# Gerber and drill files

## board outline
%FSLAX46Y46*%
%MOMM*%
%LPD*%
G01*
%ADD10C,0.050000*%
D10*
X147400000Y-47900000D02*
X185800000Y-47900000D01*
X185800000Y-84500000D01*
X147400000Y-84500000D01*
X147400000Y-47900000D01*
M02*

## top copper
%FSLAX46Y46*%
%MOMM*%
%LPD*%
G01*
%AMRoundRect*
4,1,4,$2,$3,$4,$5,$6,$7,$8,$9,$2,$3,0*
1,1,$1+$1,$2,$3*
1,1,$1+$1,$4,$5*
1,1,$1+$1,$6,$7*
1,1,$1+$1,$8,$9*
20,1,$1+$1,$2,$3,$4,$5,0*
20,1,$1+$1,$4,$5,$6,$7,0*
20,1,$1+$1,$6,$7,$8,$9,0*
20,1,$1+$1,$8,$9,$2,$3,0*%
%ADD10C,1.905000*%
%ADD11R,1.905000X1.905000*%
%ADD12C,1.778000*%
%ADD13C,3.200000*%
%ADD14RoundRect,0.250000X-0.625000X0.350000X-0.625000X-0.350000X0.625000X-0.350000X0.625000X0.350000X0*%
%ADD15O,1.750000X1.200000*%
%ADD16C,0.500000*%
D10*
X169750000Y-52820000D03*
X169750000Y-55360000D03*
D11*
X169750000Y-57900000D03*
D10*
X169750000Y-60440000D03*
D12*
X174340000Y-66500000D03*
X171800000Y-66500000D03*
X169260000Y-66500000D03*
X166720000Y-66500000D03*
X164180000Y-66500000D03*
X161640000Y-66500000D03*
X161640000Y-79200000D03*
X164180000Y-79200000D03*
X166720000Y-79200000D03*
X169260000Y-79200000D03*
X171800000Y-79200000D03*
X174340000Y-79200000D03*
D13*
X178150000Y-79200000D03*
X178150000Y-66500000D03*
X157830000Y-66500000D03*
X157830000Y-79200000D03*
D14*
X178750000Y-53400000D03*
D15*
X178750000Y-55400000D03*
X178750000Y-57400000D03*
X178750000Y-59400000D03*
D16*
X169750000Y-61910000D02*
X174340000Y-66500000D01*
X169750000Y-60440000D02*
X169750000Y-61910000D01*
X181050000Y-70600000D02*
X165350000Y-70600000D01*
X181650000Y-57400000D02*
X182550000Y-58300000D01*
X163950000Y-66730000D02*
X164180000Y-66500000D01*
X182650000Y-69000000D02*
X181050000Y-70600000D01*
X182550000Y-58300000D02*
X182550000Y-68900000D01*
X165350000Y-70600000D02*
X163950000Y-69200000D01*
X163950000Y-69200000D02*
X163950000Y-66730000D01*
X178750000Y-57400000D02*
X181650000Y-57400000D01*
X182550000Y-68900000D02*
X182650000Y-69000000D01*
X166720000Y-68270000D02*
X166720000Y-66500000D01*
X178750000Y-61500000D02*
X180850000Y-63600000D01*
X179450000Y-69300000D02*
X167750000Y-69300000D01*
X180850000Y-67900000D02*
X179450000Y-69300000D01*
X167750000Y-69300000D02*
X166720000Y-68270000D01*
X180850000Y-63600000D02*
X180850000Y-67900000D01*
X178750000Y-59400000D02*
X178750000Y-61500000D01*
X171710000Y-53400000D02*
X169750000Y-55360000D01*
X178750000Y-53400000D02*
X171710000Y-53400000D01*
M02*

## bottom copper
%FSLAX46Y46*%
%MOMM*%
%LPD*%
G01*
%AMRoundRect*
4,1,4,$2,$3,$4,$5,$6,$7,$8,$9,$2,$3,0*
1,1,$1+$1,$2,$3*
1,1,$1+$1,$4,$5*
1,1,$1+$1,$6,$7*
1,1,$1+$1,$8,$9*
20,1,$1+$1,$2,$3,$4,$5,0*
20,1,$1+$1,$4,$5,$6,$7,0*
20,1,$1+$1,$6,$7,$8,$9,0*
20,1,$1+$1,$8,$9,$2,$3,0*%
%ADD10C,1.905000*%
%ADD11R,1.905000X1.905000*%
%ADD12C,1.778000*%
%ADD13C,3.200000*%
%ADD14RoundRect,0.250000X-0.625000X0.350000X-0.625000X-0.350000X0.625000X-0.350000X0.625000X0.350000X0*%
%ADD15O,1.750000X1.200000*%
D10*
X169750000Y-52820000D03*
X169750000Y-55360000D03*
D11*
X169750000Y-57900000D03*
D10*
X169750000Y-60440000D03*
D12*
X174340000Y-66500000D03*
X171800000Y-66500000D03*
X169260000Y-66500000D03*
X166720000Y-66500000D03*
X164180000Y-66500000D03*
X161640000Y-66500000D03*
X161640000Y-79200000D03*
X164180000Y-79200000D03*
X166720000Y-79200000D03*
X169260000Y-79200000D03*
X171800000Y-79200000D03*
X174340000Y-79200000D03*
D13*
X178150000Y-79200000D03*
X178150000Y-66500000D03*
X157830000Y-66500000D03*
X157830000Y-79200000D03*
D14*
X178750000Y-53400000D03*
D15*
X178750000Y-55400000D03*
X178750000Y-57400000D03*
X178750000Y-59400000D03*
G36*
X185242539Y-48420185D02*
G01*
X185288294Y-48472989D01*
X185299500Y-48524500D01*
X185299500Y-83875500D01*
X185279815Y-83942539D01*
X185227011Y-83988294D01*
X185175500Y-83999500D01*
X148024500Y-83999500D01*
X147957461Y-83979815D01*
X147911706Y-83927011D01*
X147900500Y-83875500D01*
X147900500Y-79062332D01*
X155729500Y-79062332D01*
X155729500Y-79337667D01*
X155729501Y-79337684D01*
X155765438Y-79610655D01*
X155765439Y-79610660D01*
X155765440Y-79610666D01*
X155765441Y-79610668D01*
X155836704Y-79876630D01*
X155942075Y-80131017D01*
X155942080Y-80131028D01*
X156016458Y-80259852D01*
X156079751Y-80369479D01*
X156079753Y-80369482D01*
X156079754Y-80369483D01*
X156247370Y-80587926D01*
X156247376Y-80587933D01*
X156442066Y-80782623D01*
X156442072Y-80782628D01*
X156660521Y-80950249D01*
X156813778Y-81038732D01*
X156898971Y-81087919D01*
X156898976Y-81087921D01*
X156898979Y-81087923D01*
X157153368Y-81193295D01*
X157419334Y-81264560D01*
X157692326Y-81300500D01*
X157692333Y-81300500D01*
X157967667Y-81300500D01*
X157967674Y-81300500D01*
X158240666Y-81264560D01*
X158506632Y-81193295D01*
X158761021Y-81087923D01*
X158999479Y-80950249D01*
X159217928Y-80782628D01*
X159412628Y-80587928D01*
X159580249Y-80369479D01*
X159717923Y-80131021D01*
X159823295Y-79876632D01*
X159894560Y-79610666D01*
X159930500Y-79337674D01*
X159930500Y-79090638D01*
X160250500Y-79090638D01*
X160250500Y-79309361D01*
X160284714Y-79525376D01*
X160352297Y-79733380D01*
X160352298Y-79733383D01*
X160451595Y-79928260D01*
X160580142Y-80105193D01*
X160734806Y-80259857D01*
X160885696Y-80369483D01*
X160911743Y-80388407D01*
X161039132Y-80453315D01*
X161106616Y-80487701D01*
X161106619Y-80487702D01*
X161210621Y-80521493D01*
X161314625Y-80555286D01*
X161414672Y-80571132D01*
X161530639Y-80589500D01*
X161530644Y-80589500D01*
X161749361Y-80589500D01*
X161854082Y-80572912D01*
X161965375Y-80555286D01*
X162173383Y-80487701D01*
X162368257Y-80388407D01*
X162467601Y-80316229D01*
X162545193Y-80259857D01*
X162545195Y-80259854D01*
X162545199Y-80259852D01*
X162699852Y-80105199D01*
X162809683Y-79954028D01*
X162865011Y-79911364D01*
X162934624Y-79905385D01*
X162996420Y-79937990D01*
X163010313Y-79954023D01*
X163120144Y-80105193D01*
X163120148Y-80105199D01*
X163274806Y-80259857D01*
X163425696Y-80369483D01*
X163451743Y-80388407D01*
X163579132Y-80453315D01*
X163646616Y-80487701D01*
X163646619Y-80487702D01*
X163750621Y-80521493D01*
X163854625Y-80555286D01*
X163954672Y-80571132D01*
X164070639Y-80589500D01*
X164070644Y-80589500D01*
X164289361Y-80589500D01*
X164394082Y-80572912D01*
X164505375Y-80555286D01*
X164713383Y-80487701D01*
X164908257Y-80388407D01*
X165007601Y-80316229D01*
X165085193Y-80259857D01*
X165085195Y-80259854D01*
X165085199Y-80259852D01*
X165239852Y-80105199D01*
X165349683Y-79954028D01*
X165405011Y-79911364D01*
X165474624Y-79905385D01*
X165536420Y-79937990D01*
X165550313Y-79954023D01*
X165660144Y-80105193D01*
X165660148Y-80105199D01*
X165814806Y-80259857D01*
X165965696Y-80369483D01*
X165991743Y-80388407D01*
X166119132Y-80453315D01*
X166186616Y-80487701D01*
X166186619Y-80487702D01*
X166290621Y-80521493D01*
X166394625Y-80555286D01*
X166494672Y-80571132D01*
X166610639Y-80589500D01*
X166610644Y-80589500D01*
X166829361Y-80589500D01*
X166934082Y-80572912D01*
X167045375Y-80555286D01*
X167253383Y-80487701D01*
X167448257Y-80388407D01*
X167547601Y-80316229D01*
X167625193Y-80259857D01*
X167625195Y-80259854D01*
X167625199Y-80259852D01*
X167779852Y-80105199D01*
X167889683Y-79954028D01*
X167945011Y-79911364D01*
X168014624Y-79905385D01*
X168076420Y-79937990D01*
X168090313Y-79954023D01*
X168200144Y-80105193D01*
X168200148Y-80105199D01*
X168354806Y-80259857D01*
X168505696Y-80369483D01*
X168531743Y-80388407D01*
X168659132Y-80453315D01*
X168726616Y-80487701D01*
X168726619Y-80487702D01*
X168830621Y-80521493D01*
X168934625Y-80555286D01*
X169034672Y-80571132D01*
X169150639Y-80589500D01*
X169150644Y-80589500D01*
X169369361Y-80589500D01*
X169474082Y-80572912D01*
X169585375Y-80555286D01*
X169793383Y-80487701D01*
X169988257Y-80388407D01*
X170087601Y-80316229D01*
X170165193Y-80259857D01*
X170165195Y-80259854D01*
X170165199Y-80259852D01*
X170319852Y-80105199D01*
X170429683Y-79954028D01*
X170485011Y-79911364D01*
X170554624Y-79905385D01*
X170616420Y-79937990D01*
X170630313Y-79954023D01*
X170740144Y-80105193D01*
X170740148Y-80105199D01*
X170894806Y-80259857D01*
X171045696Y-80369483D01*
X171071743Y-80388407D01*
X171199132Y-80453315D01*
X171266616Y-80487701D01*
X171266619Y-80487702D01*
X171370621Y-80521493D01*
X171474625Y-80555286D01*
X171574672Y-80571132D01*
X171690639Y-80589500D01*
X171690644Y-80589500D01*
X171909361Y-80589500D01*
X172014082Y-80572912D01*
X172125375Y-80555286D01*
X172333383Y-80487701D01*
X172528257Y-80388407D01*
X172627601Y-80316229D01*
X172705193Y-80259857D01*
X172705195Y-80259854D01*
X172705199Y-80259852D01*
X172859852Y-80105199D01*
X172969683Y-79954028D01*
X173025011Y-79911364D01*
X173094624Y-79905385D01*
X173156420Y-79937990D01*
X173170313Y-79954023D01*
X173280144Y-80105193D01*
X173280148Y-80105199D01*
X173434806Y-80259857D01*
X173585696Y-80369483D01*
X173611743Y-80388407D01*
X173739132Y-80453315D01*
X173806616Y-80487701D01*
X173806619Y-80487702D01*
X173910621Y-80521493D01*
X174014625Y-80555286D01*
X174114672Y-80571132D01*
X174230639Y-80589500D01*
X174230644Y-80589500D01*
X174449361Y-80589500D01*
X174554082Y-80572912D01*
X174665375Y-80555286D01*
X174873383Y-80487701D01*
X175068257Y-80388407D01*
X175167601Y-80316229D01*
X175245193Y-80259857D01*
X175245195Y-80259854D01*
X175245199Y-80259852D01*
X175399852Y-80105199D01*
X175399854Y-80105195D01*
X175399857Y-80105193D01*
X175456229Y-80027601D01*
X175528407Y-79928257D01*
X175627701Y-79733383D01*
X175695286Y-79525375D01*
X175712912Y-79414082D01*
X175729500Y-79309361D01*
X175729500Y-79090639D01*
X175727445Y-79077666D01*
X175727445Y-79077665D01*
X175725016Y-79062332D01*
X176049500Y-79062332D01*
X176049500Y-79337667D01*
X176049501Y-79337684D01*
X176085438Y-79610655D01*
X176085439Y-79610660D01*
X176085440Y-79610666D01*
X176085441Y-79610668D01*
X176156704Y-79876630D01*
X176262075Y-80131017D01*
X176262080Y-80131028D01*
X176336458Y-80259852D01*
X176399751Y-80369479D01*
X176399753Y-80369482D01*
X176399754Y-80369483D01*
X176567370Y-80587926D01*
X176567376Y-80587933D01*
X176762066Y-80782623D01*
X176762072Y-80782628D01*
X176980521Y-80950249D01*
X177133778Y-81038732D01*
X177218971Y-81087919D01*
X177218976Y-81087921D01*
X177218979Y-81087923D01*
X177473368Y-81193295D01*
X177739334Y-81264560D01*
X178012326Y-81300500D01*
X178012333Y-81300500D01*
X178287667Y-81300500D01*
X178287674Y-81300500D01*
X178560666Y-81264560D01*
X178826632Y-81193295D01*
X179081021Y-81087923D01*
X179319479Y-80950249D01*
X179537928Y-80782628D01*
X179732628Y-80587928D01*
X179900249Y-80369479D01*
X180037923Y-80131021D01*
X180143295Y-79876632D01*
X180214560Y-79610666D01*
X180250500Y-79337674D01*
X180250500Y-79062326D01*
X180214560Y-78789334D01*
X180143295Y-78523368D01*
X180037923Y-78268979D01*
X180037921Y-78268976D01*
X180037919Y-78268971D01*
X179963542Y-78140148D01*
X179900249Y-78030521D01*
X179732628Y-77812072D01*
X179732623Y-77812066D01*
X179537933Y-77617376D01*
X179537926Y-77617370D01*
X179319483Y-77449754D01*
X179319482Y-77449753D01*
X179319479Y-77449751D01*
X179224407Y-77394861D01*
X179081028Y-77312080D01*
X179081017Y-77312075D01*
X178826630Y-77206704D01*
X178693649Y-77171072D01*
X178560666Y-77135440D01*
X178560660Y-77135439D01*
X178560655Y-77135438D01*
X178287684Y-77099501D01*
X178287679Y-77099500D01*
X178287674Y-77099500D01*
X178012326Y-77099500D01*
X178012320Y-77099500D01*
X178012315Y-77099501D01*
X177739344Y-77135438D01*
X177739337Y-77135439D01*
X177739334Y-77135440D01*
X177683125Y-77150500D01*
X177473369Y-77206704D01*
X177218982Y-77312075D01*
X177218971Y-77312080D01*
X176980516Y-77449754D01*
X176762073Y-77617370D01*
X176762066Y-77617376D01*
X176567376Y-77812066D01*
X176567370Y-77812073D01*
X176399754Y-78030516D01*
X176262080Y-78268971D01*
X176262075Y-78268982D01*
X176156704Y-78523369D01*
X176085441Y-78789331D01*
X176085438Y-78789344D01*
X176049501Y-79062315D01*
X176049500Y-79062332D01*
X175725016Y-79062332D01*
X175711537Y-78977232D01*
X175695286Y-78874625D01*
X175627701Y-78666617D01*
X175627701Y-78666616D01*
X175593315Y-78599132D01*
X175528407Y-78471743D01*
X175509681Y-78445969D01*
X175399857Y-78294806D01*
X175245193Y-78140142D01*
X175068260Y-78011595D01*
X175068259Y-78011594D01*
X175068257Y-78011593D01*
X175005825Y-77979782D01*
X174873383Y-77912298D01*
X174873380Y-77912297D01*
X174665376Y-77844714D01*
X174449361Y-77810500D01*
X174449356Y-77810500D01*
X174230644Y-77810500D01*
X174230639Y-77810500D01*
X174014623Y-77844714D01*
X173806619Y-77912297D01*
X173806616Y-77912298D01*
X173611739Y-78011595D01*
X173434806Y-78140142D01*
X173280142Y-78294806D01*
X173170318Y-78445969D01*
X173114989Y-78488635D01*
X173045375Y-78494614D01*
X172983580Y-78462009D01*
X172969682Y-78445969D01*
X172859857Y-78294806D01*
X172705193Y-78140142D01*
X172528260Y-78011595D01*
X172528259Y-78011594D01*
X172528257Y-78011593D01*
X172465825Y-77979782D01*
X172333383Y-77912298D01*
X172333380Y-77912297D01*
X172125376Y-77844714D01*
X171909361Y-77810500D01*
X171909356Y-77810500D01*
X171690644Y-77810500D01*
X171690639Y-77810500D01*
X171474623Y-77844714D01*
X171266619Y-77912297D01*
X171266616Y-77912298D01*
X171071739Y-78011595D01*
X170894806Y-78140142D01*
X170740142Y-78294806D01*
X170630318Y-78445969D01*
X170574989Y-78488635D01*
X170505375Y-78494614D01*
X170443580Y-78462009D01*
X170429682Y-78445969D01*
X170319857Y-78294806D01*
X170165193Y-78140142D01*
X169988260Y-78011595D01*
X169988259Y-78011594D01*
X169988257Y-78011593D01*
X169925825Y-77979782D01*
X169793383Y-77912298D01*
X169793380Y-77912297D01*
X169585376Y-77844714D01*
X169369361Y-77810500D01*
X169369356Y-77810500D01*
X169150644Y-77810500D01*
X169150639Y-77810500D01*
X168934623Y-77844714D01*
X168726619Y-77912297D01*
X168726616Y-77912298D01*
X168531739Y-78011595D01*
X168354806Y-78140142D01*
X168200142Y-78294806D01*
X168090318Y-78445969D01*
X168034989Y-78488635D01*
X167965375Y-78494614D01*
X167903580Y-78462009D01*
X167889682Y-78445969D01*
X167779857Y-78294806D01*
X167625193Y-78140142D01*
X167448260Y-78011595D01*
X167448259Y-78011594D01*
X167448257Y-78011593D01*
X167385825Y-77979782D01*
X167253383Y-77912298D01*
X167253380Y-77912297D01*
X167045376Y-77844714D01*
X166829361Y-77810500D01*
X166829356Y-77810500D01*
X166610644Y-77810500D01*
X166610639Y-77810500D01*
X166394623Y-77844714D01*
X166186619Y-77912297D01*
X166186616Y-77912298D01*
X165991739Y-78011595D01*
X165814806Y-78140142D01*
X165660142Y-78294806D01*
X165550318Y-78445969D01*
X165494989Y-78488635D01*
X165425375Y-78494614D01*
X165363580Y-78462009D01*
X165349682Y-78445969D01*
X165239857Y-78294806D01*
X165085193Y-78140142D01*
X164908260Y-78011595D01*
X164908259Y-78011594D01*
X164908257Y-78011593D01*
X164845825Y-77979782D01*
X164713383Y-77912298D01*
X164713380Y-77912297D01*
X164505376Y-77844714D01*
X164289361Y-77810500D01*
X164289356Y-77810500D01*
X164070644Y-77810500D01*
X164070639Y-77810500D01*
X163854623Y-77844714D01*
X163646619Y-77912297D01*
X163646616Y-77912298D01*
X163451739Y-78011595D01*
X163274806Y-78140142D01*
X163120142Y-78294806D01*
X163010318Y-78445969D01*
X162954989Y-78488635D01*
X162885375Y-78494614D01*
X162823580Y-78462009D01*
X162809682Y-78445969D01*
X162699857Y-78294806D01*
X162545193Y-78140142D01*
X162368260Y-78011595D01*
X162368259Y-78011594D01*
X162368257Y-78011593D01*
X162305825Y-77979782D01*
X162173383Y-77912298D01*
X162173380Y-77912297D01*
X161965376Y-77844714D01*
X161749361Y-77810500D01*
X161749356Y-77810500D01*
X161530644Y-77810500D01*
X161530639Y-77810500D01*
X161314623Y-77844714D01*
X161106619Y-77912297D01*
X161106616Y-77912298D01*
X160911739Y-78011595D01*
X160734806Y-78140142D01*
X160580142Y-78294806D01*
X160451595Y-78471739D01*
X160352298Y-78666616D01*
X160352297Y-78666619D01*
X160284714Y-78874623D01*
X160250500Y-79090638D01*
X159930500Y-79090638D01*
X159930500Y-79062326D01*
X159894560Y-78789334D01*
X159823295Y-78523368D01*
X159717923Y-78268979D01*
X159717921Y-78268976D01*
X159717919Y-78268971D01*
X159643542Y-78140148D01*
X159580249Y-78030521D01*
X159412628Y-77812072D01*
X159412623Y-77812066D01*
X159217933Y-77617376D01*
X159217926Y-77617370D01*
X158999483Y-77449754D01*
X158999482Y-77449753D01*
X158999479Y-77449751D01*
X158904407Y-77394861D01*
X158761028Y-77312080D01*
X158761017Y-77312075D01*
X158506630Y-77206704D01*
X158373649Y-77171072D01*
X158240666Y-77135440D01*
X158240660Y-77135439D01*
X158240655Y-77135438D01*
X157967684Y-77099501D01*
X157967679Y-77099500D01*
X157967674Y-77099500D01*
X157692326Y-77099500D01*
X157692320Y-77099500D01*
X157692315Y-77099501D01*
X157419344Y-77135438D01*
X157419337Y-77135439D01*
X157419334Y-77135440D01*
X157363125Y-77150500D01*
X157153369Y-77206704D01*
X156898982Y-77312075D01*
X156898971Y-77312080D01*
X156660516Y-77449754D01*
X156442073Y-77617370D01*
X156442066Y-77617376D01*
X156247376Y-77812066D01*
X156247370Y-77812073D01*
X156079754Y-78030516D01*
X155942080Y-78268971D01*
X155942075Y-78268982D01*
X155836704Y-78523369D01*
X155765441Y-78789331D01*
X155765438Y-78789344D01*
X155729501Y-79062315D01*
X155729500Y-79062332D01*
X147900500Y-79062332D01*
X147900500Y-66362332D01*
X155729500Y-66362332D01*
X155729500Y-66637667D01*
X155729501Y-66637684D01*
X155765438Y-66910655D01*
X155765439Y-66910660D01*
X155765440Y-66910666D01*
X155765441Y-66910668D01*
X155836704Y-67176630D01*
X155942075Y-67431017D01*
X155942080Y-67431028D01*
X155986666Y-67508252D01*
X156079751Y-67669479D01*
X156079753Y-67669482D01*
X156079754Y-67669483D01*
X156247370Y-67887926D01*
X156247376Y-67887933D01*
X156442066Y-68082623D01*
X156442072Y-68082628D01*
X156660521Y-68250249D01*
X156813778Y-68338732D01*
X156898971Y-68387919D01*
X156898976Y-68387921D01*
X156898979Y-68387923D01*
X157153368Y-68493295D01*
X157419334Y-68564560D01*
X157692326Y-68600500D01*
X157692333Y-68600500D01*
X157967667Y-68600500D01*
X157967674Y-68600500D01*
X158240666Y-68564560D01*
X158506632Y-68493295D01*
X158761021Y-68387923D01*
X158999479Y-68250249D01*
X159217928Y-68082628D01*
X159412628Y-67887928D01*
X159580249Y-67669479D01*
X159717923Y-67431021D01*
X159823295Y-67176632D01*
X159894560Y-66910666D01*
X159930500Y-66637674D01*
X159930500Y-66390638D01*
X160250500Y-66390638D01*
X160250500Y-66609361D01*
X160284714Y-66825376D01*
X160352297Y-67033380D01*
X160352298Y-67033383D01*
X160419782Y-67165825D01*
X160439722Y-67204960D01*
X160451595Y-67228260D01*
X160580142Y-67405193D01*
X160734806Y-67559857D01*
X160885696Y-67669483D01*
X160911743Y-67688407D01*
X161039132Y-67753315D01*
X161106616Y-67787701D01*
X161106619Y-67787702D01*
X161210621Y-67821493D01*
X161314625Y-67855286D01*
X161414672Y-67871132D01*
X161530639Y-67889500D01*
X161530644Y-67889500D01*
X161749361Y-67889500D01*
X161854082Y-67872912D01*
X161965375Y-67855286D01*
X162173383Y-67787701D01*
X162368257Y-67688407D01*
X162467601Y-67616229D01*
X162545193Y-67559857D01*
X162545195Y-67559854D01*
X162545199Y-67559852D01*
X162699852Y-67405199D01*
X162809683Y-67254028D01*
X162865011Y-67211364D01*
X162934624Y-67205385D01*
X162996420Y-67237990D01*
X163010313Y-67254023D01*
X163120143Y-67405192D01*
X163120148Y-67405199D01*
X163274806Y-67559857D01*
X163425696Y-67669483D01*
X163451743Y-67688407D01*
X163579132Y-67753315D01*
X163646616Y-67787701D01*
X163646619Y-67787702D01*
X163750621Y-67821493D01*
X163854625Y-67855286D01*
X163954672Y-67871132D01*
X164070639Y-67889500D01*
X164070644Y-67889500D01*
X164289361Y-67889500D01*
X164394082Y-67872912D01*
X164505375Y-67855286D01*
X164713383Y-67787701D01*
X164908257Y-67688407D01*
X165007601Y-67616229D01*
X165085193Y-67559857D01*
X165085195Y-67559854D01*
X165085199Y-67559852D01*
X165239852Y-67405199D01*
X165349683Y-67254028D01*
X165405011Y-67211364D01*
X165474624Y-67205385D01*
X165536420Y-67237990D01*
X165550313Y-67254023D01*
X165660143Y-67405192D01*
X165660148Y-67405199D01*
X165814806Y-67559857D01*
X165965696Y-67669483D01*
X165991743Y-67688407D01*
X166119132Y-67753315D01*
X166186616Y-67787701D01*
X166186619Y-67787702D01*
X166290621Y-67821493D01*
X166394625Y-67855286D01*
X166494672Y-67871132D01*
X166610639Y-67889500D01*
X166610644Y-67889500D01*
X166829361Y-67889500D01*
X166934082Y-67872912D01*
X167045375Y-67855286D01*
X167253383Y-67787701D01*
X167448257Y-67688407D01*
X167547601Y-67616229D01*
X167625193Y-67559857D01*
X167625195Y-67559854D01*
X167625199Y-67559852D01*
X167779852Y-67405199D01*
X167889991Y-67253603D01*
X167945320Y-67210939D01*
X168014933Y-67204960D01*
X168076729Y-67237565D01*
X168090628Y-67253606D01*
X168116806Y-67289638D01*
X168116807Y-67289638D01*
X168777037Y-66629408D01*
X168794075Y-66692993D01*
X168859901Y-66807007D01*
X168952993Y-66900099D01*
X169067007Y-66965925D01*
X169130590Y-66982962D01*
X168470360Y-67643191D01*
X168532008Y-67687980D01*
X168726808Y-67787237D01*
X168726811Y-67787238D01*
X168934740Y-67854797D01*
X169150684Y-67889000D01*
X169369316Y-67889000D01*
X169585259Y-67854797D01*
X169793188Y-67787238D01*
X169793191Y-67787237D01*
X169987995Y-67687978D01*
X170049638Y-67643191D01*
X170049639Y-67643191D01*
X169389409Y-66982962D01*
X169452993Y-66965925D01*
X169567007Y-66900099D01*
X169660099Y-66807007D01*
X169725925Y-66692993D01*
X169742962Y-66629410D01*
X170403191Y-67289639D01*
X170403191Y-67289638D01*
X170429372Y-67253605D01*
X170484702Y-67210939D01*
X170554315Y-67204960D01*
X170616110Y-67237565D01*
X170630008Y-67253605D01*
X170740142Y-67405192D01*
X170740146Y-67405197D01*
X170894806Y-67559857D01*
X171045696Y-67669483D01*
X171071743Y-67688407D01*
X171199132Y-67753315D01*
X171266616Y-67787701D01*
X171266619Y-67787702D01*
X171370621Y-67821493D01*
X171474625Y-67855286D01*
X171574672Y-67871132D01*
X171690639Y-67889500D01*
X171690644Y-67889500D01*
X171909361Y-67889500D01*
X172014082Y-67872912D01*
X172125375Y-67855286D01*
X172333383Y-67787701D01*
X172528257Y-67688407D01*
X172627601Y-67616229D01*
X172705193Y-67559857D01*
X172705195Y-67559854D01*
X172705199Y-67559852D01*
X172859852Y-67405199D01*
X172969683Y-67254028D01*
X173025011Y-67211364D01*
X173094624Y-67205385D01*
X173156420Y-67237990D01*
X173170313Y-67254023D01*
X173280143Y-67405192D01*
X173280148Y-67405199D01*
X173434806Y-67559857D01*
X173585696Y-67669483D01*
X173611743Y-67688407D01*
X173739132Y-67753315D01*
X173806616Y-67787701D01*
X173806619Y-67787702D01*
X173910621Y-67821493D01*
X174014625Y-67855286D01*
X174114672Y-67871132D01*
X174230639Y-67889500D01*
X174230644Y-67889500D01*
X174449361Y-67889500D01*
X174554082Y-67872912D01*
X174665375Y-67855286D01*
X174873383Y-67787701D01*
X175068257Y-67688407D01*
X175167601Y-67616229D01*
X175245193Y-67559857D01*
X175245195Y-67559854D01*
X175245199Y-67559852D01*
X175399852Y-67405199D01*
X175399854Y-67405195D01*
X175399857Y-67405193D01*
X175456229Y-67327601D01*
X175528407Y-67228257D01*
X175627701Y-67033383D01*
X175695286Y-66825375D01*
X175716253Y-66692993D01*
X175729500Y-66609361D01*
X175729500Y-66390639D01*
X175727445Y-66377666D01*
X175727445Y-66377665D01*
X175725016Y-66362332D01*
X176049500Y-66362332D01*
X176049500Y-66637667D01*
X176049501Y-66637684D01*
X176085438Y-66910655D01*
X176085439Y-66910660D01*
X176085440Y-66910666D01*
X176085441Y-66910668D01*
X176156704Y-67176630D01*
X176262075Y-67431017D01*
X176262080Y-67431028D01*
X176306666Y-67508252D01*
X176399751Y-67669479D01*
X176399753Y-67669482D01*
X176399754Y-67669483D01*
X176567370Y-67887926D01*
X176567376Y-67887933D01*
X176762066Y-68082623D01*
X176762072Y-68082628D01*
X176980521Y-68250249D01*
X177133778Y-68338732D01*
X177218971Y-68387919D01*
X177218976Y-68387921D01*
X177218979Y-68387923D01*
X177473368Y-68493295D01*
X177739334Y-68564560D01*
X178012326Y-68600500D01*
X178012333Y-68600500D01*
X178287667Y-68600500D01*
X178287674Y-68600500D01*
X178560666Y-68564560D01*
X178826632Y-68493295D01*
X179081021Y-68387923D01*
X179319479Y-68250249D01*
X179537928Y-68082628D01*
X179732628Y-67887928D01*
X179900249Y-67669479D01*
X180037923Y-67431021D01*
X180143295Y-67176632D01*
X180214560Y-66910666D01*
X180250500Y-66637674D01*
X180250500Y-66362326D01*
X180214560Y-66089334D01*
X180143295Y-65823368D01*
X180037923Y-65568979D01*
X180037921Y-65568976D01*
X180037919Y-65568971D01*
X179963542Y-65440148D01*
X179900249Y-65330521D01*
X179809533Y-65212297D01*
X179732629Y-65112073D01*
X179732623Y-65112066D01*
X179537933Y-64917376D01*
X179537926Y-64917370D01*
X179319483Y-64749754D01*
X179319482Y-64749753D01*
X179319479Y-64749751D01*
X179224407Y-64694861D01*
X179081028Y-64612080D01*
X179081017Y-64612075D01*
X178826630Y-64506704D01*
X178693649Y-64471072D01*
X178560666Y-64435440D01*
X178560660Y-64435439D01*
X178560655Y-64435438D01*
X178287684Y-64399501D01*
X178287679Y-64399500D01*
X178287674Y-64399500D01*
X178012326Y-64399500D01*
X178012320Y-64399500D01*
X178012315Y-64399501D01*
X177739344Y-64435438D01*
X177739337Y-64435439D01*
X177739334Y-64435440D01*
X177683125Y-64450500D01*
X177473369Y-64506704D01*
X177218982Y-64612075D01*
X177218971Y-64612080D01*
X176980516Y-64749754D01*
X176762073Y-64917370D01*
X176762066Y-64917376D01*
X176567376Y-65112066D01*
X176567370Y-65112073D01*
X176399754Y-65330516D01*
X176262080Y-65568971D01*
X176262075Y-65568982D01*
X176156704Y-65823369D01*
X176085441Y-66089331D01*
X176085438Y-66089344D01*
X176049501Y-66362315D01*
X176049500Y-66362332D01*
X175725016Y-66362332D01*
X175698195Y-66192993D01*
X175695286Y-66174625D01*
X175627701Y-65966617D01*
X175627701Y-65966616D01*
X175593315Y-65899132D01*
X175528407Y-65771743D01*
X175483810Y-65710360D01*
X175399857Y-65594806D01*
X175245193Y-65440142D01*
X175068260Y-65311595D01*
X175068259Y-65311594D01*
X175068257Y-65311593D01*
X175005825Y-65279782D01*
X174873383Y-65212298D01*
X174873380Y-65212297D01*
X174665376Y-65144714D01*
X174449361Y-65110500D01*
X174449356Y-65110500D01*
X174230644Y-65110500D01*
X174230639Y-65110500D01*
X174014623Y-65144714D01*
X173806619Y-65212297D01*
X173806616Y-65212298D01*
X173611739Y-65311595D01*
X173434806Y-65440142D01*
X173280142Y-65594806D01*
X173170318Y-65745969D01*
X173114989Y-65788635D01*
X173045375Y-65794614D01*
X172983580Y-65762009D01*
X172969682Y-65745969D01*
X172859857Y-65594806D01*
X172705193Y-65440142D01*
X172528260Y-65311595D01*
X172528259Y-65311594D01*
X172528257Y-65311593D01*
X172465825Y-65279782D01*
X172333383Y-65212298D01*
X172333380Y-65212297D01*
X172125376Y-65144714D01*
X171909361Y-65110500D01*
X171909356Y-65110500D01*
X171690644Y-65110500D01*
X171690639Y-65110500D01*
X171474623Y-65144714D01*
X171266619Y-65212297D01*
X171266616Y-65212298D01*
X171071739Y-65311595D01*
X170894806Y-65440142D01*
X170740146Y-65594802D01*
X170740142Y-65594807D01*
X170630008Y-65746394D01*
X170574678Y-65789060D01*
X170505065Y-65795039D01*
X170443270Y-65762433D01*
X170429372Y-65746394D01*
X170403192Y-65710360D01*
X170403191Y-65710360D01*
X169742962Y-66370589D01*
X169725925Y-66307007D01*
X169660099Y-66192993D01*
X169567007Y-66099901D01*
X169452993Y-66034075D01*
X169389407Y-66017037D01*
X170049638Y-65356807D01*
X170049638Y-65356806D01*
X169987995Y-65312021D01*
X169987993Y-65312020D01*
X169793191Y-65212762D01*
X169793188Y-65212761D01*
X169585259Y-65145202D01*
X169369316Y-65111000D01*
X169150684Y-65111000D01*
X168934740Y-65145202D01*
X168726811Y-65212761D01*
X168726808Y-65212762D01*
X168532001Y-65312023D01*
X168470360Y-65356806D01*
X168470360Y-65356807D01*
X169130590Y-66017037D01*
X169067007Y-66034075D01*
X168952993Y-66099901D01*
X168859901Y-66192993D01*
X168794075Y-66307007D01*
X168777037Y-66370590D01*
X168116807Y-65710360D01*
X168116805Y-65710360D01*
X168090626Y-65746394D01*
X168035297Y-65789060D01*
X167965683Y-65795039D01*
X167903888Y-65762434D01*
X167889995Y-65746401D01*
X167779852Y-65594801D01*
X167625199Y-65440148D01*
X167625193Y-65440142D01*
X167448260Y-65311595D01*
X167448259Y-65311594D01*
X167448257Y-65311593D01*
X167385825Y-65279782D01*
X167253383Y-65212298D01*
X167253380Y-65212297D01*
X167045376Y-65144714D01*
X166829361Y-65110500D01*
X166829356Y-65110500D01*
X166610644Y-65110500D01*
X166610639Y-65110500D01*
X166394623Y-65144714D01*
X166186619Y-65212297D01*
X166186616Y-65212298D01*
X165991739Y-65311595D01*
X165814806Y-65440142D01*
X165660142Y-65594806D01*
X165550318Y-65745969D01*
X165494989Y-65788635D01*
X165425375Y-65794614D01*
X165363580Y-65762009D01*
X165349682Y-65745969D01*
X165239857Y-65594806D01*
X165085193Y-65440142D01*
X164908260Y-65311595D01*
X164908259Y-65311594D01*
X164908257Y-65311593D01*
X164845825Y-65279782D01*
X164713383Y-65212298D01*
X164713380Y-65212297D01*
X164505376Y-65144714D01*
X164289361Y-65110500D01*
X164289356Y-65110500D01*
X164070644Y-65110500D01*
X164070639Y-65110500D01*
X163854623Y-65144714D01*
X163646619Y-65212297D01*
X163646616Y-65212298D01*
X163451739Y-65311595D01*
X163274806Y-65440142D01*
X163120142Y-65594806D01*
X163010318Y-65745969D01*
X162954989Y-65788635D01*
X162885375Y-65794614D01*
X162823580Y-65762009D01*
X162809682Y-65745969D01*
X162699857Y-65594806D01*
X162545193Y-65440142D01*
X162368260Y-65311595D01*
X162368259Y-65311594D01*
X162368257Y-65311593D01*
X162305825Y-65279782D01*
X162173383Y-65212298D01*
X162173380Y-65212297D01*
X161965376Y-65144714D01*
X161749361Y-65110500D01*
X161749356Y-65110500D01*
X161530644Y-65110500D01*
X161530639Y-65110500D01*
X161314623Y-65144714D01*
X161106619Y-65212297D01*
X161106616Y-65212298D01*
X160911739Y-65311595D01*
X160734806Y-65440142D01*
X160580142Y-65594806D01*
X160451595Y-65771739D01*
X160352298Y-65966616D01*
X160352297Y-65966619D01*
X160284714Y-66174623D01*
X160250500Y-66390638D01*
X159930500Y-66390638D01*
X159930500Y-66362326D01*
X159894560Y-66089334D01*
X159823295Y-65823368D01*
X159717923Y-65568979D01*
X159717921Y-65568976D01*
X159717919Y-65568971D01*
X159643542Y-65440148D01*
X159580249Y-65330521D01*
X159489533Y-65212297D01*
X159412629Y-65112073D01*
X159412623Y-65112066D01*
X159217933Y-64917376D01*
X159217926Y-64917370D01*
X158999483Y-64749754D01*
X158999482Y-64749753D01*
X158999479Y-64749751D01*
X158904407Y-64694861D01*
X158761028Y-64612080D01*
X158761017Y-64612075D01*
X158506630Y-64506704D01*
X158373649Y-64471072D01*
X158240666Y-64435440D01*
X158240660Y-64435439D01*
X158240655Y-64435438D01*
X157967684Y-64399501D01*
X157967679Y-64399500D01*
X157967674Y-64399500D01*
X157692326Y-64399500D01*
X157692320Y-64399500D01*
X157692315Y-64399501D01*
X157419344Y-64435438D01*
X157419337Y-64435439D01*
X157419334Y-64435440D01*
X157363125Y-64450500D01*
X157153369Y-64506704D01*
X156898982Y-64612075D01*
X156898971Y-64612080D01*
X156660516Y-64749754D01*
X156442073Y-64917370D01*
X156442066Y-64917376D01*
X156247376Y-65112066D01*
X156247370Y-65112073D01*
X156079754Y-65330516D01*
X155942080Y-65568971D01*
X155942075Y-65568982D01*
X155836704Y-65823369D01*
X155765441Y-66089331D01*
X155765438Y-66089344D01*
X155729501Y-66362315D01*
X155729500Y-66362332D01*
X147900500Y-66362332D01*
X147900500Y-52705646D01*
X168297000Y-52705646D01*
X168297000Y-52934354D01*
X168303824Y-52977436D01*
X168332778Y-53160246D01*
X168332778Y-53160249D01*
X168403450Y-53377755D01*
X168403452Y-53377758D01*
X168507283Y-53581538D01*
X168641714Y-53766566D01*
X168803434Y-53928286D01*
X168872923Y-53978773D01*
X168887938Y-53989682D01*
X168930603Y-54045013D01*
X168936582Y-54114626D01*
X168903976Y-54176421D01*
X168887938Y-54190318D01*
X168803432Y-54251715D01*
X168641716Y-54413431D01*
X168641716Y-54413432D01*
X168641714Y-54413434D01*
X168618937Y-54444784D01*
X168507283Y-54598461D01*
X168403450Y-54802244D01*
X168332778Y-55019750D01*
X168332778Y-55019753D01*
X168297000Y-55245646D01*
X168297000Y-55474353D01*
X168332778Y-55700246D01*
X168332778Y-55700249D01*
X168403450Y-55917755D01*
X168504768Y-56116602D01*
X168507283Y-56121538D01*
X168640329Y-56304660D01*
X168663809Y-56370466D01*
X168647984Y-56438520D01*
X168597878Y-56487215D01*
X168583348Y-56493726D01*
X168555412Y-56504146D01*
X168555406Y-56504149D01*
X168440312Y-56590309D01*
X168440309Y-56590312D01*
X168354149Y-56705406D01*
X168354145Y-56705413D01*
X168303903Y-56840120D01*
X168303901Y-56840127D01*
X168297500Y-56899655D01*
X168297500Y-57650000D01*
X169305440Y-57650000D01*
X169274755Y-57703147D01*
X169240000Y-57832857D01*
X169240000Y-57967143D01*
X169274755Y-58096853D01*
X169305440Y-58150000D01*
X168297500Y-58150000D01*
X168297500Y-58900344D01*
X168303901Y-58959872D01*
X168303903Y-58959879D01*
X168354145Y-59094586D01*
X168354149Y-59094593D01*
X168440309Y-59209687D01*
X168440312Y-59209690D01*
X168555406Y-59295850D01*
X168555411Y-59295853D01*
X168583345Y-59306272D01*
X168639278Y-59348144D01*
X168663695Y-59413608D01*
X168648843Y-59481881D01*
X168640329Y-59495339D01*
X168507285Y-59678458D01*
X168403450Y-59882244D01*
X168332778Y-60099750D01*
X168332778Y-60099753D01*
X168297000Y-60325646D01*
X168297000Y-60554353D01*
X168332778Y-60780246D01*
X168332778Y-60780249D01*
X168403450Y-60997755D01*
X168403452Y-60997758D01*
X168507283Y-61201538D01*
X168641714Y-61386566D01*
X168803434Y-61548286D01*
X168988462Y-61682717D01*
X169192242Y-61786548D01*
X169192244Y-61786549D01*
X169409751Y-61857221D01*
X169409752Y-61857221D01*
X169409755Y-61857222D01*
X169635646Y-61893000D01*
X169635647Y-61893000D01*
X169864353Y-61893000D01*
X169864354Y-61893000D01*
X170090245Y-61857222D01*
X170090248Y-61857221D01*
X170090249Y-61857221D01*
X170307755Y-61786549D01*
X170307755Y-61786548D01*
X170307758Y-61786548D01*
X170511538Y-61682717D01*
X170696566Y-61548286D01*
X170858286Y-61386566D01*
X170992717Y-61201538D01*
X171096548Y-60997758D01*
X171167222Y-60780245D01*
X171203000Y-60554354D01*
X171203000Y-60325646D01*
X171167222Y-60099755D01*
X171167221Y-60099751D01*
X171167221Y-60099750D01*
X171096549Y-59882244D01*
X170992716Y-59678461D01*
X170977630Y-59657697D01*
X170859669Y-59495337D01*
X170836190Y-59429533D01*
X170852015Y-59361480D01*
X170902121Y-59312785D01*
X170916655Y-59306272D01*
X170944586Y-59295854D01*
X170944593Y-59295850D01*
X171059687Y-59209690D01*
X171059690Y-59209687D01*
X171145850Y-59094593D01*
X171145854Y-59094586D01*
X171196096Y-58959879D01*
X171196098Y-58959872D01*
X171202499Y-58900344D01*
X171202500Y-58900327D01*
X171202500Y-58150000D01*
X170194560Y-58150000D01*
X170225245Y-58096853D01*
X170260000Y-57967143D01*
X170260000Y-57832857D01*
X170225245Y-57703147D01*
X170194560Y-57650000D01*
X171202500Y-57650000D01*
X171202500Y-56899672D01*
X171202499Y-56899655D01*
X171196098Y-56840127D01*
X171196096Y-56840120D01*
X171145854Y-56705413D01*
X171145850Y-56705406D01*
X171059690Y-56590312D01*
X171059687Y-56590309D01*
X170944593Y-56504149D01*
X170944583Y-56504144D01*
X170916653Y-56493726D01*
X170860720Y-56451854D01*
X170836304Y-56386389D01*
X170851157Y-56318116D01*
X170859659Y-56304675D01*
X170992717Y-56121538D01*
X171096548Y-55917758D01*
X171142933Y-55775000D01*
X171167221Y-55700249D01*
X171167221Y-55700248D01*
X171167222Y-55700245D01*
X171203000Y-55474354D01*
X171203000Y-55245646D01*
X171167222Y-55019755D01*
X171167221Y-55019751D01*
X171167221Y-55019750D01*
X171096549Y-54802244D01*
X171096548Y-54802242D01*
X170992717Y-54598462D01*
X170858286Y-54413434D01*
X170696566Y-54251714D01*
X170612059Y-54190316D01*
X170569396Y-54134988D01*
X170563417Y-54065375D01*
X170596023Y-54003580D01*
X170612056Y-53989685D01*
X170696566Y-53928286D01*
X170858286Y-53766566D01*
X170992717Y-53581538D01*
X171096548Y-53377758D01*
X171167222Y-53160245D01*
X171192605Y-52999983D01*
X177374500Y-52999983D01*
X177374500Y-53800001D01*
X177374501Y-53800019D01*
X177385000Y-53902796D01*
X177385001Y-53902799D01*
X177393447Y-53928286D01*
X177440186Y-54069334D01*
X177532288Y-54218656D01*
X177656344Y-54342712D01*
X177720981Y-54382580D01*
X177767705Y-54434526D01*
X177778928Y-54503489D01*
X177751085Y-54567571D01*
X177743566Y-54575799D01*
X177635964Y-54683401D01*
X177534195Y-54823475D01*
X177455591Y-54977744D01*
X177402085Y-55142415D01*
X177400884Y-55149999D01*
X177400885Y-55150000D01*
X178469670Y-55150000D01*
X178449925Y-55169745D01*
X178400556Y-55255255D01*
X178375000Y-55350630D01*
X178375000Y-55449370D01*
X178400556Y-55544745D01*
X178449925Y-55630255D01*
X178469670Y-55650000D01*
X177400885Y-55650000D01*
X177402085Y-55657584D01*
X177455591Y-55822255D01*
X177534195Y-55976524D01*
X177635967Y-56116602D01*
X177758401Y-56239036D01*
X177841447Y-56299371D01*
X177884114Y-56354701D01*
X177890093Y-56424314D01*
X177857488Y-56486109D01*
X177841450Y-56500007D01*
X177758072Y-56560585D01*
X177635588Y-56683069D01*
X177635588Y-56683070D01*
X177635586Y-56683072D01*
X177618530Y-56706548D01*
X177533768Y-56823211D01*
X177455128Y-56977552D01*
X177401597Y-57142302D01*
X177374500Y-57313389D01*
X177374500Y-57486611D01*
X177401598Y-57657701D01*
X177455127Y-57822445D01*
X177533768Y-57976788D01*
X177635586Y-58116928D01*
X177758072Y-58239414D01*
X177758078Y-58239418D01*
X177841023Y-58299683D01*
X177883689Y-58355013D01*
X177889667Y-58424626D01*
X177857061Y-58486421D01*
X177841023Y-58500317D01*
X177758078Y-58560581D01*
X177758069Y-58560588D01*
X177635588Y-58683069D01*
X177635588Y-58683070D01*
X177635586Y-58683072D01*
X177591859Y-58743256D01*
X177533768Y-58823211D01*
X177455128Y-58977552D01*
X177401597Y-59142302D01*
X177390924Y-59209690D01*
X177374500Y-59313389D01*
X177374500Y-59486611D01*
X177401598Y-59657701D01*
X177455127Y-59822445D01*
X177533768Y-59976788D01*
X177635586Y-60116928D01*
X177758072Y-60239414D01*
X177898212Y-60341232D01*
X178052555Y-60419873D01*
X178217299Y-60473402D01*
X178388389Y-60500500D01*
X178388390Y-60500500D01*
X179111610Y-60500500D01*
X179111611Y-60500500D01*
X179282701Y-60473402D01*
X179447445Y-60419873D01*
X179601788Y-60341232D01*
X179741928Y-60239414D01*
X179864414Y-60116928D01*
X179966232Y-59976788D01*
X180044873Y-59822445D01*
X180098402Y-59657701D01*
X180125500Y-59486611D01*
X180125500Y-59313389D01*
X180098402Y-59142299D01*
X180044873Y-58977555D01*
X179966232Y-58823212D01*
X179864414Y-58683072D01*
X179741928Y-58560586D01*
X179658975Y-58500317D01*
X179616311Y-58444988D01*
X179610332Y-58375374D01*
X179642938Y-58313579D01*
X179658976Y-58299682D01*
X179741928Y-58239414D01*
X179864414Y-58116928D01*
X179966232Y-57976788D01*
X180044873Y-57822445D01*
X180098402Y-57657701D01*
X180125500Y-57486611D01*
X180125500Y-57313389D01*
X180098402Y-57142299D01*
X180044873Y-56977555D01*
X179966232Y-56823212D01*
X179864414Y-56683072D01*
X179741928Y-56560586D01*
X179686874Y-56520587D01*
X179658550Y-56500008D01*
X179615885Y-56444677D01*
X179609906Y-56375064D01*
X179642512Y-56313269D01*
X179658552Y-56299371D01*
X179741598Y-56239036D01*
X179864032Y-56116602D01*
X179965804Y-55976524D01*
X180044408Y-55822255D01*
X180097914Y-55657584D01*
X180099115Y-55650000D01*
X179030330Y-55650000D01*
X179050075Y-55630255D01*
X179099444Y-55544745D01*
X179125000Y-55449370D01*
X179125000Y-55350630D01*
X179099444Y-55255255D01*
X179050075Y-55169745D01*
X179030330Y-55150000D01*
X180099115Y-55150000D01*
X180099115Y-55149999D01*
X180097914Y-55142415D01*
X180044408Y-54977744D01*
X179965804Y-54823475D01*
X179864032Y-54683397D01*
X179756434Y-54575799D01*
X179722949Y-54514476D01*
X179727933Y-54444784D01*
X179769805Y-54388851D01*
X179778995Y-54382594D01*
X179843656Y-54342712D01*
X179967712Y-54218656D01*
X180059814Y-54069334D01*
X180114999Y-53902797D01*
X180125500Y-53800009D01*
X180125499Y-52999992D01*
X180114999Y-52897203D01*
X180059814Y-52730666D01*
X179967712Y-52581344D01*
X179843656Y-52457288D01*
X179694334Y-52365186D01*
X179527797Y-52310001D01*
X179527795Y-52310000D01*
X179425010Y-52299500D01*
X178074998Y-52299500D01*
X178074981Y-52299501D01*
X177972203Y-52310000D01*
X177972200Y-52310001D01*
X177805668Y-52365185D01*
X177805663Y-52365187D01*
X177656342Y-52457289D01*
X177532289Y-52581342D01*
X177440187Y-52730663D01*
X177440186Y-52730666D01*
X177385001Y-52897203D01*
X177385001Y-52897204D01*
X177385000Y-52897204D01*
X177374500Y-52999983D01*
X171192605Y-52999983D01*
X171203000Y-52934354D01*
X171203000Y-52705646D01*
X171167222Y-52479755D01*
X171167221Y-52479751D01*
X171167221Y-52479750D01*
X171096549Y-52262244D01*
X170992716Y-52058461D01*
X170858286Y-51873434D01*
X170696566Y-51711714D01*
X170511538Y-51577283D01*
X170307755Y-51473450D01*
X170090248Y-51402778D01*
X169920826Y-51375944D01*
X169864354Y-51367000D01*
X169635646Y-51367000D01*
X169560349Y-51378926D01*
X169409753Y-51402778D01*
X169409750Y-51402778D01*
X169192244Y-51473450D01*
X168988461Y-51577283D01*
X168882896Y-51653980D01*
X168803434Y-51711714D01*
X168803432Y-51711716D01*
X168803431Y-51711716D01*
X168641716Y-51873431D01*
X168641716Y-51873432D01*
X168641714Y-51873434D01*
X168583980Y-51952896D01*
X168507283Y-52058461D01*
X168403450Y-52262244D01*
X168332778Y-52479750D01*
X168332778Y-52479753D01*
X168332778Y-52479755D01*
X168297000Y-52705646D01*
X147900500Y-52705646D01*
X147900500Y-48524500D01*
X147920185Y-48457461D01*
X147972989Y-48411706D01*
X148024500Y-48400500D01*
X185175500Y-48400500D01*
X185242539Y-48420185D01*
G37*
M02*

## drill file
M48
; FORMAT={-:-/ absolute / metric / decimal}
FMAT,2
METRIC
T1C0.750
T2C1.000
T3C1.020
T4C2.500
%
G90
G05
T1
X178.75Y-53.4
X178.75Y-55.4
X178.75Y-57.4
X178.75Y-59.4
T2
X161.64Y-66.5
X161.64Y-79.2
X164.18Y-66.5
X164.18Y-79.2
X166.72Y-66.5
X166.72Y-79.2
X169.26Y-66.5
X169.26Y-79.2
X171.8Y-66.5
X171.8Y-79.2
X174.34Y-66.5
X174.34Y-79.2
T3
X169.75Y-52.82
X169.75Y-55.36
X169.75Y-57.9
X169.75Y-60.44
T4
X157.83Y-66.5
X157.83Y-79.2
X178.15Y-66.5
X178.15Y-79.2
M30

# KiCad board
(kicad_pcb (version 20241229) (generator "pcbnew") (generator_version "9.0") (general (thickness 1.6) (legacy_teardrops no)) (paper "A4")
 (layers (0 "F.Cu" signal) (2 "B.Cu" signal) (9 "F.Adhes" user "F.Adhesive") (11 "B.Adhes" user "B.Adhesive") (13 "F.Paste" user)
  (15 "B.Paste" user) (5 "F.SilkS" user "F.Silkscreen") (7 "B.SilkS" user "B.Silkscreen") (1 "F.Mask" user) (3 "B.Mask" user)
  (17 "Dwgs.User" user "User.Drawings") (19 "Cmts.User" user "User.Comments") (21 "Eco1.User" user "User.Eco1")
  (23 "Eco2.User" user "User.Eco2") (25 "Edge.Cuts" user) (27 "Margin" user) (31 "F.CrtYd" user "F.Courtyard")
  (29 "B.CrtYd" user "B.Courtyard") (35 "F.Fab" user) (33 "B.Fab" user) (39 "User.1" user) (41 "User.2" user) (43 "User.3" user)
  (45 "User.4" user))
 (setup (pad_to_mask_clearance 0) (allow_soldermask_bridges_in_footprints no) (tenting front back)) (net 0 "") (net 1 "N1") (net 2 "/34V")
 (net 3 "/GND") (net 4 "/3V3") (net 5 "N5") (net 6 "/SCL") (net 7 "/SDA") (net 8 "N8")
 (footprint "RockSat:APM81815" (layer "F.Cu") (at 151.92 61.75 90)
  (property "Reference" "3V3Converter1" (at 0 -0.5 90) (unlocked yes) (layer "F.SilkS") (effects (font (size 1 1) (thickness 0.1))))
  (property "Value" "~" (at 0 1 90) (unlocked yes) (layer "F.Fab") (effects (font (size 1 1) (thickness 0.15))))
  (pad "1" thru_hole circle (at 8.93 17.83 90) (size 1.905 1.905) (drill 1.02) (layers "*.Cu" "*.Mask") (remove_unused_layers no)
   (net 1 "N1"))
  (pad "2" thru_hole circle (at 6.39 17.83 90) (size 1.905 1.905) (drill 1.02) (layers "*.Cu" "*.Mask") (remove_unused_layers no)
   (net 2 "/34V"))
  (pad "3" thru_hole rect (at 3.85 17.83 90) (size 1.905 1.905) (drill 1.02) (layers "*.Cu" "*.Mask") (remove_unused_layers no)
   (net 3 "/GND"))
  (pad "4" thru_hole circle (at 1.31 17.83 90) (size 1.905 1.905) (drill 1.02) (layers "*.Cu" "*.Mask") (remove_unused_layers no)
   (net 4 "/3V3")))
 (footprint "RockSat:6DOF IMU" (layer "F.Cu") (at 167.99 72.85 180)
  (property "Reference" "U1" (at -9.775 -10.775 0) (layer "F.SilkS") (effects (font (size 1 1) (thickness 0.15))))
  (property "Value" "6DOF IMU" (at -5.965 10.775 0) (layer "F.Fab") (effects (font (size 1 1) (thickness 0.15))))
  (pad "JP1_1" thru_hole circle (at -6.35 6.35 180) (size 1.778 1.778) (drill 1) (layers "*.Cu" "*.Mask") (remove_unused_layers no)
   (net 4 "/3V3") (solder_mask_margin 0.102))
  (pad "JP1_2" thru_hole circle (at -3.81 6.35 180) (size 1.778 1.778) (drill 1) (layers "*.Cu" "*.Mask") (remove_unused_layers no)
   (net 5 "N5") (solder_mask_margin 0.102))
  (pad "JP1_3" thru_hole circle (at -1.27 6.35 180) (size 1.778 1.778) (drill 1) (layers "*.Cu" "*.Mask") (remove_unused_layers no)
   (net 3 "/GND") (solder_mask_margin 0.102))
  (pad "JP1_4" thru_hole circle (at 1.27 6.35 180) (size 1.778 1.778) (drill 1) (layers "*.Cu" "*.Mask") (remove_unused_layers no)
   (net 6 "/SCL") (solder_mask_margin 0.102))
  (pad "JP1_5" thru_hole circle (at 3.81 6.35 180) (size 1.778 1.778) (drill 1) (layers "*.Cu" "*.Mask") (remove_unused_layers no)
   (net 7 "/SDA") (solder_mask_margin 0.102))
  (pad "JP1_6" thru_hole circle (at 6.35 6.35 180) (size 1.778 1.778) (drill 1) (layers "*.Cu" "*.Mask") (remove_unused_layers no)
   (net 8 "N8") (solder_mask_margin 0.102))
  (pad "JP3_1" thru_hole circle (at 6.35 -6.35 180) (size 1.778 1.778) (drill 1) (layers "*.Cu" "*.Mask") (remove_unused_layers no)
   (solder_mask_margin 0.102))
  (pad "JP3_2" thru_hole circle (at 3.81 -6.35 180) (size 1.778 1.778) (drill 1) (layers "*.Cu" "*.Mask") (remove_unused_layers no)
   (solder_mask_margin 0.102))
  (pad "JP3_3" thru_hole circle (at 1.27 -6.35 180) (size 1.778 1.778) (drill 1) (layers "*.Cu" "*.Mask") (remove_unused_layers no)
   (solder_mask_margin 0.102))
  (pad "JP3_4" thru_hole circle (at -1.27 -6.35 180) (size 1.778 1.778) (drill 1) (layers "*.Cu" "*.Mask") (remove_unused_layers no)
   (solder_mask_margin 0.102))
  (pad "JP3_5" thru_hole circle (at -3.81 -6.35 180) (size 1.778 1.778) (drill 1) (layers "*.Cu" "*.Mask") (remove_unused_layers no)
   (solder_mask_margin 0.102))
  (pad "JP3_6" thru_hole circle (at -6.35 -6.35 180) (size 1.778 1.778) (drill 1) (layers "*.Cu" "*.Mask") (remove_unused_layers no)
   (solder_mask_margin 0.102))
  (pad "SH1" thru_hole circle (at -10.16 -6.35 180) (size 3.2 3.2) (drill 2.5) (layers "*.Cu" "*.Mask") (remove_unused_layers no)
   (solder_mask_margin 0.102))
  (pad "SH2" thru_hole circle (at -10.16 6.35 180) (size 3.2 3.2) (drill 2.5) (layers "*.Cu" "*.Mask") (remove_unused_layers no)
   (solder_mask_margin 0.102))
  (pad "SH3" thru_hole circle (at 10.16 6.35 180) (size 3.2 3.2) (drill 2.5) (layers "*.Cu" "*.Mask") (remove_unused_layers no)
   (solder_mask_margin 0.102))
  (pad "SH4" thru_hole circle (at 10.16 -6.35 180) (size 3.2 3.2) (drill 2.5) (layers "*.Cu" "*.Mask") (remove_unused_layers no)
   (solder_mask_margin 0.102)))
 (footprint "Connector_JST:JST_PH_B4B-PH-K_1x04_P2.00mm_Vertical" (layer "F.Cu") (at 178.75 53.4 -90)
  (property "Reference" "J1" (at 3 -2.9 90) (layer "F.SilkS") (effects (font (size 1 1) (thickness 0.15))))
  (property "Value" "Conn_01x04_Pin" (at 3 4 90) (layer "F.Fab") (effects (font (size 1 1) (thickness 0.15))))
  (pad "1" thru_hole roundrect (at 0 0 270) (size 1.2 1.75) (drill 0.75) (layers "*.Cu" "*.Mask") (remove_unused_layers no)
   (roundrect_rratio 0.208333) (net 2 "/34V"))
  (pad "2" thru_hole oval (at 2 0 270) (size 1.2 1.75) (drill 0.75) (layers "*.Cu" "*.Mask") (remove_unused_layers no) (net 3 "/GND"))
  (pad "3" thru_hole oval (at 4 0 270) (size 1.2 1.75) (drill 0.75) (layers "*.Cu" "*.Mask") (remove_unused_layers no) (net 7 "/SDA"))
  (pad "4" thru_hole oval (at 6 0 270) (size 1.2 1.75) (drill 0.75) (layers "*.Cu" "*.Mask") (remove_unused_layers no) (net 6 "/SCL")))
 (gr_rect (start 147.4 47.9) (end 185.8 84.5) (stroke (width 0.05) (type default)) (fill no) (layer "Edge.Cuts"))
 (segment (start 169.75 61.91) (end 174.34 66.5) (width 0.5) (layer "F.Cu") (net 4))
 (segment (start 169.75 60.44) (end 169.75 61.91) (width 0.5) (layer "F.Cu") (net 4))
 (segment (start 181.05 70.6) (end 165.35 70.6) (width 0.5) (layer "F.Cu") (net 7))
 (segment (start 181.65 57.4) (end 182.55 58.3) (width 0.5) (layer "F.Cu") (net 7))
 (segment (start 163.95 66.73) (end 164.18 66.5) (width 0.5) (layer "F.Cu") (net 7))
 (segment (start 182.65 69) (end 181.05 70.6) (width 0.5) (layer "F.Cu") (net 7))
 (segment (start 182.55 58.3) (end 182.55 68.9) (width 0.5) (layer "F.Cu") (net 7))
 (segment (start 165.35 70.6) (end 163.95 69.2) (width 0.5) (layer "F.Cu") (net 7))
 (segment (start 163.95 69.2) (end 163.95 66.73) (width 0.5) (layer "F.Cu") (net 7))
 (segment (start 178.75 57.4) (end 181.65 57.4) (width 0.5) (layer "F.Cu") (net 7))
 (segment (start 182.55 68.9) (end 182.65 69) (width 0.5) (layer "F.Cu") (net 7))
 (segment (start 166.72 68.27) (end 166.72 66.5) (width 0.5) (layer "F.Cu") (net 6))
 (segment (start 178.75 61.5) (end 180.85 63.6) (width 0.5) (layer "F.Cu") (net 6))
 (segment (start 179.45 69.3) (end 167.75 69.3) (width 0.5) (layer "F.Cu") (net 6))
 (segment (start 180.85 67.9) (end 179.45 69.3) (width 0.5) (layer "F.Cu") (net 6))
 (segment (start 167.75 69.3) (end 166.72 68.27) (width 0.5) (layer "F.Cu") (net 6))
 (segment (start 180.85 63.6) (end 180.85 67.9) (width 0.5) (layer "F.Cu") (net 6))
 (segment (start 178.75 59.4) (end 178.75 61.5) (width 0.5) (layer "F.Cu") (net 6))
 (segment (start 171.71 53.4) (end 169.75 55.36) (width 0.5) (layer "F.Cu") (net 2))
 (segment (start 178.75 53.4) (end 171.71 53.4) (width 0.5) (layer "F.Cu") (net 2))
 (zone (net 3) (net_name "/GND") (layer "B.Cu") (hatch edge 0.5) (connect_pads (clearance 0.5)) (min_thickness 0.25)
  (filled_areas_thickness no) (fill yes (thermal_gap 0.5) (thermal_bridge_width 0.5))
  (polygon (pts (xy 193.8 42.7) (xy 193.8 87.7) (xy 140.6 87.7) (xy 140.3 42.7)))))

